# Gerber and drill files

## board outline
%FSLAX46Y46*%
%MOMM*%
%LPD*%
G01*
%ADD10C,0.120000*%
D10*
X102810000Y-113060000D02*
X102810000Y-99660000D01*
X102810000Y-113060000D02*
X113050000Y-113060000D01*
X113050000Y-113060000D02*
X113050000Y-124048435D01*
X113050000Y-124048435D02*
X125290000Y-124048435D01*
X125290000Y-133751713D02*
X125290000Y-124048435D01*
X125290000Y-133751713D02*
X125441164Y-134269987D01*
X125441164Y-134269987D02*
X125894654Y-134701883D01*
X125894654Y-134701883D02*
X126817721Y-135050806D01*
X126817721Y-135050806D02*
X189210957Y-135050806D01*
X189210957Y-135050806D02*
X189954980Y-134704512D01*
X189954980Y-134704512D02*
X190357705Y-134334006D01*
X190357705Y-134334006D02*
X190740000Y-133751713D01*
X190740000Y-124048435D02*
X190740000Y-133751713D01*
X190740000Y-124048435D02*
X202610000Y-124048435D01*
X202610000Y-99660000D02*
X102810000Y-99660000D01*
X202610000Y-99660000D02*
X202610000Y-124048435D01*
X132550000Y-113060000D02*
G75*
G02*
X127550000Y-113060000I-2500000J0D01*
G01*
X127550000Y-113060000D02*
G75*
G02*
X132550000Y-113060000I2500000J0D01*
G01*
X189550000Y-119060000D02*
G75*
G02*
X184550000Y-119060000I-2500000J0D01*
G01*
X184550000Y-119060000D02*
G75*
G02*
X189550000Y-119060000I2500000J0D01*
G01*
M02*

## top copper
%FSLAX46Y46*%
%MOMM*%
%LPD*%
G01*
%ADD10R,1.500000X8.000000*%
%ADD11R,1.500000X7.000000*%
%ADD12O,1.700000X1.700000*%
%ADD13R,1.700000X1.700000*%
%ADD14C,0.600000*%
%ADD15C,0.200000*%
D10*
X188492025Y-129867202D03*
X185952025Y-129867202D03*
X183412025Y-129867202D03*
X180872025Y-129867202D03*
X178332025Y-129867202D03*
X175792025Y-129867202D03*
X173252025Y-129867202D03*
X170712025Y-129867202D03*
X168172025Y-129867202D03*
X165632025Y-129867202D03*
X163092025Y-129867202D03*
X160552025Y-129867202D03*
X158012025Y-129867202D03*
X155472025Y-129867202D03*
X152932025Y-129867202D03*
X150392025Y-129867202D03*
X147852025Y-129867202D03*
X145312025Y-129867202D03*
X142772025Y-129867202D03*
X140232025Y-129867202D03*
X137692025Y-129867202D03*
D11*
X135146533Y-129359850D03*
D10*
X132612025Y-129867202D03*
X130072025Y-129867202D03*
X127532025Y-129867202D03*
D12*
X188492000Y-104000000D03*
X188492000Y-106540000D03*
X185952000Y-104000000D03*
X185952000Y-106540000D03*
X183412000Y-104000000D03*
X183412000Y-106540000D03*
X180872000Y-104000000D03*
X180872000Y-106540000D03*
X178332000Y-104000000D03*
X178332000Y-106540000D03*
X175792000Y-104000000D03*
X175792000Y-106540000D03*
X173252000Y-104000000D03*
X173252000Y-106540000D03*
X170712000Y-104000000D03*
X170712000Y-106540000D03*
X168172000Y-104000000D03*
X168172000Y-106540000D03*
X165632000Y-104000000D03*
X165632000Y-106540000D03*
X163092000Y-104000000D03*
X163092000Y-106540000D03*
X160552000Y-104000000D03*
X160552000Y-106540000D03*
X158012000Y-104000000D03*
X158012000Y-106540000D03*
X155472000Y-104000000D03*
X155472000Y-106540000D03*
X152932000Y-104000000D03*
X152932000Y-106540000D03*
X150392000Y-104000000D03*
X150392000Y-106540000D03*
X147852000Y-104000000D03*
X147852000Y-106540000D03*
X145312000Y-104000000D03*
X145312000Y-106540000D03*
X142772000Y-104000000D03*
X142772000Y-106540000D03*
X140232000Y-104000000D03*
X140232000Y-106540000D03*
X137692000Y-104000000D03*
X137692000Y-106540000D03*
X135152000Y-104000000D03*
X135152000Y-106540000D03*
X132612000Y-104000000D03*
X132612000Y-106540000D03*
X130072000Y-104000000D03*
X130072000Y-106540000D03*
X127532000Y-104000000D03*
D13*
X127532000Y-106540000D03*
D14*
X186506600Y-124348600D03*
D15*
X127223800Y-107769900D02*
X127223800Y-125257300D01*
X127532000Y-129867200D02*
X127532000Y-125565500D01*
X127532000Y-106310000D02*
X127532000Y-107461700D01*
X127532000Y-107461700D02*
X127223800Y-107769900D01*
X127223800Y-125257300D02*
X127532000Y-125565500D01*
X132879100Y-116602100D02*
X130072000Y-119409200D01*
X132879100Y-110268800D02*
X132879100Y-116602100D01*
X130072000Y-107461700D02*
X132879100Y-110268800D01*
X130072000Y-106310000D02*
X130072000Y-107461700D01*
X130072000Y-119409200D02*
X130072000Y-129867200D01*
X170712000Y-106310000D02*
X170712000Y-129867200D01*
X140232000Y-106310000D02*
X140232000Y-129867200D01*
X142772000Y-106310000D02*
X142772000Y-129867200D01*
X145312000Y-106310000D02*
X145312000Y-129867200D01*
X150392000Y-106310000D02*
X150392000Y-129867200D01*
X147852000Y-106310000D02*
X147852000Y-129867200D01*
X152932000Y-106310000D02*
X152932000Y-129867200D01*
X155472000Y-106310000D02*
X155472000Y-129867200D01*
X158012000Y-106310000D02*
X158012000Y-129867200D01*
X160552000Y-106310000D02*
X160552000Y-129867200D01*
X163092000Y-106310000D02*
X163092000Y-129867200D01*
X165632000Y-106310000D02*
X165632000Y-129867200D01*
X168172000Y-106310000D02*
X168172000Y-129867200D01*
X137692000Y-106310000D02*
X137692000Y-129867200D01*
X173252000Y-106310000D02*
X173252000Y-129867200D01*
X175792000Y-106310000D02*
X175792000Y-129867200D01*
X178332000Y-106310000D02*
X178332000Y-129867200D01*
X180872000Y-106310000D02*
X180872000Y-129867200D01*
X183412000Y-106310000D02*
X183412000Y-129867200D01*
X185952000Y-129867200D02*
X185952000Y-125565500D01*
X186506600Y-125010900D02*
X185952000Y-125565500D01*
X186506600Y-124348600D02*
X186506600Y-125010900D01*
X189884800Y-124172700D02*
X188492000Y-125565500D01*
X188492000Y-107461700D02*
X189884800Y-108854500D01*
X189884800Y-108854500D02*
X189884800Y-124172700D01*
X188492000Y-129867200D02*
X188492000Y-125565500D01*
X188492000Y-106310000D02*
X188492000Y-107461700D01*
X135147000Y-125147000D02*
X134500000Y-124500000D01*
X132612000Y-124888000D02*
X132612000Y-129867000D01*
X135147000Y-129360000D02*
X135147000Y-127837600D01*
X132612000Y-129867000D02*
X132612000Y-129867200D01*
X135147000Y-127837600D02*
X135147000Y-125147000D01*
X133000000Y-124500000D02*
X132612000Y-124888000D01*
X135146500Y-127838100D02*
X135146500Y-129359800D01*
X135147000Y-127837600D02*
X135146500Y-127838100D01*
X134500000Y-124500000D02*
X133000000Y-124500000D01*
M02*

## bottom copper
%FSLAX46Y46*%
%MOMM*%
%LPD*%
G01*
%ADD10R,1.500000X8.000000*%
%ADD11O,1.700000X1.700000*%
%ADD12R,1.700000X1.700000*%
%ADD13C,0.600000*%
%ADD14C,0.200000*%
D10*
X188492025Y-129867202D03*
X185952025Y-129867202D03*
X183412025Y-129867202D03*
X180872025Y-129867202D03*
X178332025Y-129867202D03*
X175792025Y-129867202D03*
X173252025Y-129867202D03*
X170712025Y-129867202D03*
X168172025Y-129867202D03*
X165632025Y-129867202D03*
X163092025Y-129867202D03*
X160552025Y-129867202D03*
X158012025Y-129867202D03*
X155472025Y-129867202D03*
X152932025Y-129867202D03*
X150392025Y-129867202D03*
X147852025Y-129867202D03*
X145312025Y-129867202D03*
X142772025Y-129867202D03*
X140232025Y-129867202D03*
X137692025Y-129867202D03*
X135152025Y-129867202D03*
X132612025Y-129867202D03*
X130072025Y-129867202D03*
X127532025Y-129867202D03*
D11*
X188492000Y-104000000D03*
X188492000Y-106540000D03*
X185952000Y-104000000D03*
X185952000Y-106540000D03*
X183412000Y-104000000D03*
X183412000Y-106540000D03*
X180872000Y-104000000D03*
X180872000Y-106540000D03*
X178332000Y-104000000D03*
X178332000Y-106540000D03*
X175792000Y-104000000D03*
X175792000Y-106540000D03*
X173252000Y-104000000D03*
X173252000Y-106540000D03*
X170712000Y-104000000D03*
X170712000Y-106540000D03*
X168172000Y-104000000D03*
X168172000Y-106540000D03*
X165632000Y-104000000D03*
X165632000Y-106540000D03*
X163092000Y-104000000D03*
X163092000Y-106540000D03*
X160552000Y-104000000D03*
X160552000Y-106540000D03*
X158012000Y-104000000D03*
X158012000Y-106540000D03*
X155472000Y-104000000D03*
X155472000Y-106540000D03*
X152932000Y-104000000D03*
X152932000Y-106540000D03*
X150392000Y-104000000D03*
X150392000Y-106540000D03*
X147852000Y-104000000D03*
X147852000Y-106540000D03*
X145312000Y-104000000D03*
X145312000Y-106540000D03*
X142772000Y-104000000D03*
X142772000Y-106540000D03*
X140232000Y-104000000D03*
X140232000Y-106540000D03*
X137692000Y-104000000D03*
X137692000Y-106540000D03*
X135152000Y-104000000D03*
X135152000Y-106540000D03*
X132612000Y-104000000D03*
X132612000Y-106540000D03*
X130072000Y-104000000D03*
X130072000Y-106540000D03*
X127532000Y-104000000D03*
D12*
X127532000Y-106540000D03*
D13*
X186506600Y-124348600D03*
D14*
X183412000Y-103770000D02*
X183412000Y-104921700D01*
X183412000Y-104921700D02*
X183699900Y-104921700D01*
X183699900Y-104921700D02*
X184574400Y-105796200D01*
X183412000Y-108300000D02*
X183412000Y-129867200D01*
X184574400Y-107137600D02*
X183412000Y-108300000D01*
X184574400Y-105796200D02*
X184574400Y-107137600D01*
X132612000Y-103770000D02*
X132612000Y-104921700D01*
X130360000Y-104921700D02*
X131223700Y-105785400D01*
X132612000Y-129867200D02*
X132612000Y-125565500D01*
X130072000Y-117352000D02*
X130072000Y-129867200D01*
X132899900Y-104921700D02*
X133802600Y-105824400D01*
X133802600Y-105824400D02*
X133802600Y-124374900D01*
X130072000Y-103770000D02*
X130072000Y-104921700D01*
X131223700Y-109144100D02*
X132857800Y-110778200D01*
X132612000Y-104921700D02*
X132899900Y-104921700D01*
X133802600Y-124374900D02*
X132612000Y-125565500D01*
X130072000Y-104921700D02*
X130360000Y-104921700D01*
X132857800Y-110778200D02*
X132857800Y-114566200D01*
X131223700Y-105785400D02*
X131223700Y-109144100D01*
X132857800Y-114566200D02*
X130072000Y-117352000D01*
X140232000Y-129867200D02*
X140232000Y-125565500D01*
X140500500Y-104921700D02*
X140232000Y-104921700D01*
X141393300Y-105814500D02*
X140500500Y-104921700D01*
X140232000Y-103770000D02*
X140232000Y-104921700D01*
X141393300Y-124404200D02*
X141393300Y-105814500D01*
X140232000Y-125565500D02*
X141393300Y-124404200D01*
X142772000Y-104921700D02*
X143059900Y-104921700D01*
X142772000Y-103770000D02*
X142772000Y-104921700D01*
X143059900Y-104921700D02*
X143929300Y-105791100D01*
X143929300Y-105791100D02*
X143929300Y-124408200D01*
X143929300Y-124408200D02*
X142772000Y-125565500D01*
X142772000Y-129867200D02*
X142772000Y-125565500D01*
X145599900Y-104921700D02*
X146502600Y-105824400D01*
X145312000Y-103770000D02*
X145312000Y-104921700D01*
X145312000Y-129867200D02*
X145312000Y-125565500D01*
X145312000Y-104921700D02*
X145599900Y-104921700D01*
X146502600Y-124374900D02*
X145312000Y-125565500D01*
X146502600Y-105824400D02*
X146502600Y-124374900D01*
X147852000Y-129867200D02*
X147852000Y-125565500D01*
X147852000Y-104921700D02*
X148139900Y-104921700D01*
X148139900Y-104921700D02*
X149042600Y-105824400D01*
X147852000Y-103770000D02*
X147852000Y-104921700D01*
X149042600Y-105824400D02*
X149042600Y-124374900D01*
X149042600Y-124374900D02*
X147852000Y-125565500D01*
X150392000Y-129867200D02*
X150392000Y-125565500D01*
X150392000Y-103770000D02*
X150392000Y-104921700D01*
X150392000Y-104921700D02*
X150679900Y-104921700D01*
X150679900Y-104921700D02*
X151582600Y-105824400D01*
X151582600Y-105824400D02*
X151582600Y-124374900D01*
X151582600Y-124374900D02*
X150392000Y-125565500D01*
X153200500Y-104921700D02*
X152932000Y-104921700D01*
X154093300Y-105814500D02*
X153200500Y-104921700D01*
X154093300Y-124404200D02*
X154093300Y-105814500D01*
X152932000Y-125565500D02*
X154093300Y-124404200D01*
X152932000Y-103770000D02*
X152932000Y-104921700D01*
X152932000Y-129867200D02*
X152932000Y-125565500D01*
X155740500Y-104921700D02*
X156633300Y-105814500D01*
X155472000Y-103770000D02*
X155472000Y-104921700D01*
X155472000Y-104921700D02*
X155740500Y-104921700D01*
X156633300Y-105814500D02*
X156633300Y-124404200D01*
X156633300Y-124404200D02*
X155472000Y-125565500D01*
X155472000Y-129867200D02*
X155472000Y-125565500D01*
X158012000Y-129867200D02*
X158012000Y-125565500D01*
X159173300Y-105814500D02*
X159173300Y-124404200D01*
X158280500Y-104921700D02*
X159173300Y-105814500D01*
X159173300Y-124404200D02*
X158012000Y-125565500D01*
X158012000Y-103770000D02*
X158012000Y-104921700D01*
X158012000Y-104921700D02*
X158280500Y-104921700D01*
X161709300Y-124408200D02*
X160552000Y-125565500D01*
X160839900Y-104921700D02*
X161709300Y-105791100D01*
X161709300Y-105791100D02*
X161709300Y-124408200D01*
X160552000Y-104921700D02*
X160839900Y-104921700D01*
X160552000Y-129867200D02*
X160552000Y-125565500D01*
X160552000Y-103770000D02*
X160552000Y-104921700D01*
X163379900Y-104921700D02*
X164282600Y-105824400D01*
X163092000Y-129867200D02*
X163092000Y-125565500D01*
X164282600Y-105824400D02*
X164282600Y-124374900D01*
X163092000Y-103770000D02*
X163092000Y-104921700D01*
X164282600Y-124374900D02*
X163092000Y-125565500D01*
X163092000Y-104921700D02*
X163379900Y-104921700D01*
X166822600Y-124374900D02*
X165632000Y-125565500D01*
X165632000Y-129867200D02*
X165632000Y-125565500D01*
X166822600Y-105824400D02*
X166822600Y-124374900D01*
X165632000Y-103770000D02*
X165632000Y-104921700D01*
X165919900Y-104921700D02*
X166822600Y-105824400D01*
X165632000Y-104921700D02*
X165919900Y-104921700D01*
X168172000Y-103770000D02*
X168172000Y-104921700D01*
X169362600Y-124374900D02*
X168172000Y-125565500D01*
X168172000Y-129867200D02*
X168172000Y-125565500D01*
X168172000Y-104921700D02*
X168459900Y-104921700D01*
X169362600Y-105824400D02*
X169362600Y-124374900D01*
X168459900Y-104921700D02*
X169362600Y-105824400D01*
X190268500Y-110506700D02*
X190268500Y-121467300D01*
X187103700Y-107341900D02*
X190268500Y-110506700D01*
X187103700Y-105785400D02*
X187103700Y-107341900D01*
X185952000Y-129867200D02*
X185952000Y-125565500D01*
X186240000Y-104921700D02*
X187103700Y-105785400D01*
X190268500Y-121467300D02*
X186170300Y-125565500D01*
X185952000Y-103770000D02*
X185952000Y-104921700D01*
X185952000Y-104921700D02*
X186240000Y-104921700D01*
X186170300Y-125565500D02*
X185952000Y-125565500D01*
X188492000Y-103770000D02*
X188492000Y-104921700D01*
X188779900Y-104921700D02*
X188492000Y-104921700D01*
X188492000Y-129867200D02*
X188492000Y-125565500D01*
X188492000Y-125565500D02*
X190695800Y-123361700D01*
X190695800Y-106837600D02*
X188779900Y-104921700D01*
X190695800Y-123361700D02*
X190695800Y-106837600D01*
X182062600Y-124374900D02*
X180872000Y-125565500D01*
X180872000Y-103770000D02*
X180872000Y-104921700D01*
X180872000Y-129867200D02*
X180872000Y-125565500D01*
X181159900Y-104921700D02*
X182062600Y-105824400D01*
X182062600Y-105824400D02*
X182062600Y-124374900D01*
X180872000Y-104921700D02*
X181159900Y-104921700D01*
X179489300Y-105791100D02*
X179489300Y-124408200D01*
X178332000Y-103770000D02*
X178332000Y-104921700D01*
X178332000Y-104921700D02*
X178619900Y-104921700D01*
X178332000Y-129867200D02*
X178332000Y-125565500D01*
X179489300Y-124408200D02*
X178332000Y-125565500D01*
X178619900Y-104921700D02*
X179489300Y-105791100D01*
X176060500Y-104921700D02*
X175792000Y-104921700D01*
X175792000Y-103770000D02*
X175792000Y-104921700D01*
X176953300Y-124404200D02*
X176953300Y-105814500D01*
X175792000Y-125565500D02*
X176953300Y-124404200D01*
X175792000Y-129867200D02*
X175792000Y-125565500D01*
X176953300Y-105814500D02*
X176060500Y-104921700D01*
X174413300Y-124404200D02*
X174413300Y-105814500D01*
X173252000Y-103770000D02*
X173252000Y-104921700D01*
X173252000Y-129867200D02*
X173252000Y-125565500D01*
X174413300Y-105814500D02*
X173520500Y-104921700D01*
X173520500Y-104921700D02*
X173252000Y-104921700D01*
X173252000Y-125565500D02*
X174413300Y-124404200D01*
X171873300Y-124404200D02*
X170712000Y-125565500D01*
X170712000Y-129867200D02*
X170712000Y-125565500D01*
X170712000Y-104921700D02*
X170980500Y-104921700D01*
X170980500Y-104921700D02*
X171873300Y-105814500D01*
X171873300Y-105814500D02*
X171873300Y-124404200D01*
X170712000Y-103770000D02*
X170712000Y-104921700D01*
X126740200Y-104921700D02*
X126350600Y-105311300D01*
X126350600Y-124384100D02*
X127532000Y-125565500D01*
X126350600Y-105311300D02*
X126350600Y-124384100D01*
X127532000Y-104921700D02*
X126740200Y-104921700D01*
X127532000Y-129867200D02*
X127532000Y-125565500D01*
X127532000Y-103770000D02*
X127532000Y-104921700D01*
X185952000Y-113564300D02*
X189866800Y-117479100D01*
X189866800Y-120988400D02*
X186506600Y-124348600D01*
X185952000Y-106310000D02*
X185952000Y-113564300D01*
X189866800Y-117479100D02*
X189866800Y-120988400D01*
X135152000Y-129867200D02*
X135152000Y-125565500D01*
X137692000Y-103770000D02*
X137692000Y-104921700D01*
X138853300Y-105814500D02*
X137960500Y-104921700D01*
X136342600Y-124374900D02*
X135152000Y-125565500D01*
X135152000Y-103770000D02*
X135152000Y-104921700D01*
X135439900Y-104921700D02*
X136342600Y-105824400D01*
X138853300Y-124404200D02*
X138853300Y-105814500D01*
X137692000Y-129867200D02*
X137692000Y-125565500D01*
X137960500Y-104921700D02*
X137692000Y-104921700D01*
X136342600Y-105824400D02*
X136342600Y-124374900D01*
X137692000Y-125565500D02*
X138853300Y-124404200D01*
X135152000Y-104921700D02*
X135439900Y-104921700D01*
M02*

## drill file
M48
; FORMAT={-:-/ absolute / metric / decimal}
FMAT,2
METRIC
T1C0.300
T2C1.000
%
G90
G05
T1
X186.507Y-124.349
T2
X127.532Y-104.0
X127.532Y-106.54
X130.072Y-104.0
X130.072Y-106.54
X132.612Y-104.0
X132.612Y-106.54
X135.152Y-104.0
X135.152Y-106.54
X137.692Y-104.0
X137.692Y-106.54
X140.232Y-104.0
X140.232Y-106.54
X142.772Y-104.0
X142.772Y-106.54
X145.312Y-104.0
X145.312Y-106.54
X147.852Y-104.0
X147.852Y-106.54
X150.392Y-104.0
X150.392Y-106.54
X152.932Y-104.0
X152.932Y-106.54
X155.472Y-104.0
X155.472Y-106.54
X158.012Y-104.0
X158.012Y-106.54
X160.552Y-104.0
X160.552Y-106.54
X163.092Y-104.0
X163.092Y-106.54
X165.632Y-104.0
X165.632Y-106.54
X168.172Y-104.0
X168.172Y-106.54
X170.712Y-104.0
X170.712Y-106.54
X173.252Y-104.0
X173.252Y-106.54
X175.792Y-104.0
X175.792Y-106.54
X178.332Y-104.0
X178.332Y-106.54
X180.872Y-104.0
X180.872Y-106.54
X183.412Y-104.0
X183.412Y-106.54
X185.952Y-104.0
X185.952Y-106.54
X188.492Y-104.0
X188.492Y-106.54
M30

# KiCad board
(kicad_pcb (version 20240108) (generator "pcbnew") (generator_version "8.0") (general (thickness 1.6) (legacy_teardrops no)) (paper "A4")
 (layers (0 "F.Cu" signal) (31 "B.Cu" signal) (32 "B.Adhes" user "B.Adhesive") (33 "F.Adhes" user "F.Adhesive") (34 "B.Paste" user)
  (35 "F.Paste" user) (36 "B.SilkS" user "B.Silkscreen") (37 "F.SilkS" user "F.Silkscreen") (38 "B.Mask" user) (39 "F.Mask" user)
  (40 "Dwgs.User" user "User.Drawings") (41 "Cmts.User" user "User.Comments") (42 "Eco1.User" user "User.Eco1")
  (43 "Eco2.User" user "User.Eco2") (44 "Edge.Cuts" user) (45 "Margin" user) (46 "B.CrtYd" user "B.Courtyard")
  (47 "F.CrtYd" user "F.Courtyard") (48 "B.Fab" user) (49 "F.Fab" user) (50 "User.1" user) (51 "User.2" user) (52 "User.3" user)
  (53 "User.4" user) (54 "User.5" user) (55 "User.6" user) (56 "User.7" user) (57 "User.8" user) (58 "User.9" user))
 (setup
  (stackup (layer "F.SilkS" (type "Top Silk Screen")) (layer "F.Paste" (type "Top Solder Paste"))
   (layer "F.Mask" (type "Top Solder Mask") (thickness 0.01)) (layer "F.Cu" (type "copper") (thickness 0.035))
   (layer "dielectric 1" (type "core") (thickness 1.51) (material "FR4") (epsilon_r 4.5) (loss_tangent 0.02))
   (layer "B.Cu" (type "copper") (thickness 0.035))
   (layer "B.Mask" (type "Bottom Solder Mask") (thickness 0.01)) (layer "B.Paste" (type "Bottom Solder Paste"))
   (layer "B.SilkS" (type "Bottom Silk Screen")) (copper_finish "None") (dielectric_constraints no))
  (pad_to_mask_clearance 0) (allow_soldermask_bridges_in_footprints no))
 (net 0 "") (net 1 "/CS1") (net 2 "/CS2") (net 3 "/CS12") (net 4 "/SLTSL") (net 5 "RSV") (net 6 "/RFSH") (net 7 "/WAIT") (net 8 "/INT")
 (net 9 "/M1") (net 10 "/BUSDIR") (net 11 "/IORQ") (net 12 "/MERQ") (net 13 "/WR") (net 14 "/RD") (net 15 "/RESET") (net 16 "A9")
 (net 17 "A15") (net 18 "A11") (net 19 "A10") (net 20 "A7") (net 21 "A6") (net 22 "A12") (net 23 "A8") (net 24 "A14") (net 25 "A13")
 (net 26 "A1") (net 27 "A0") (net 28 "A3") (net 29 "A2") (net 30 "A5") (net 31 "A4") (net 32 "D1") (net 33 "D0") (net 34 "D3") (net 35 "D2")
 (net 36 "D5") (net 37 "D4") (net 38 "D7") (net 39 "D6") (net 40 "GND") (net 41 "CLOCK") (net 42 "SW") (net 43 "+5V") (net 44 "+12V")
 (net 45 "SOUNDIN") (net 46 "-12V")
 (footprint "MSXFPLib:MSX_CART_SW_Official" (layer "F.Cu") (at 151.71 99.66)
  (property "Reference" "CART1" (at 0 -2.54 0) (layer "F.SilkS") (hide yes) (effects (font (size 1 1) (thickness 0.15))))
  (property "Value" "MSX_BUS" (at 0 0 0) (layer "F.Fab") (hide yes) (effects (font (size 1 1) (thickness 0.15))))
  (fp_line (start -48.9 13.4) (end -48.9 0) (stroke (width 0.12) (type solid)) (layer "Edge.Cuts"))
  (fp_line (start -48.9 13.4) (end -38.66 13.4) (stroke (width 0.12) (type solid)) (layer "Edge.Cuts"))
  (fp_line (start -38.66 13.4) (end -38.66 24.388435) (stroke (width 0.12) (type solid)) (layer "Edge.Cuts"))
  (fp_line (start -38.66 24.388435) (end -26.42 24.388435) (stroke (width 0.12) (type solid)) (layer "Edge.Cuts"))
  (fp_line (start -26.42 34.091713) (end -26.42 24.388435) (stroke (width 0.12) (type solid)) (layer "Edge.Cuts"))
  (fp_line (start -26.42 34.091713) (end -26.268836 34.609987) (stroke (width 0.12) (type solid)) (layer "Edge.Cuts"))
  (fp_line (start -26.268836 34.609987) (end -25.815346 35.041883) (stroke (width 0.12) (type solid)) (layer "Edge.Cuts"))
  (fp_line (start -25.815346 35.041883) (end -24.892279 35.390806) (stroke (width 0.12) (type solid)) (layer "Edge.Cuts"))
  (fp_line (start -24.892279 35.390806) (end 37.500957 35.390806) (stroke (width 0.12) (type solid)) (layer "Edge.Cuts"))
  (fp_line (start 37.500957 35.390806) (end 38.24498 35.044512) (stroke (width 0.12) (type solid)) (layer "Edge.Cuts"))
  (fp_line (start 38.24498 35.044512) (end 38.647705 34.674006) (stroke (width 0.12) (type solid)) (layer "Edge.Cuts"))
  (fp_line (start 38.647705 34.674006) (end 39.03 34.091713) (stroke (width 0.12) (type solid)) (layer "Edge.Cuts"))
  (fp_line (start 39.03 24.388435) (end 39.03 34.091713) (stroke (width 0.12) (type solid)) (layer "Edge.Cuts"))
  (fp_line (start 39.03 24.388435) (end 50.9 24.388435) (stroke (width 0.12) (type solid)) (layer "Edge.Cuts"))
  (fp_line (start 50.9 0) (end -48.9 0) (stroke (width 0.12) (type solid)) (layer "Edge.Cuts"))
  (fp_line (start 50.9 0) (end 50.9 24.388435) (stroke (width 0.12) (type solid)) (layer "Edge.Cuts"))
  (fp_circle (center -21.66 13.4) (end -19.16 13.4) (stroke (width 0.12) (type solid)) (fill none) (layer "Edge.Cuts"))
  (fp_circle (center 35.34 19.4) (end 37.84 19.4) (stroke (width 0.12) (type solid)) (fill none) (layer "Edge.Cuts"))
  (pad "1" connect rect (at 36.782025 30.207202) (size 1.5 8) (layers "B.Cu" "B.Mask") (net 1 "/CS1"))
  (pad "2" connect rect (at 36.782025 30.207202) (size 1.5 8) (layers "F.Cu" "F.Mask") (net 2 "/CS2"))
  (pad "3" connect rect (at 34.242025 30.207202) (size 1.5 8) (layers "B.Cu" "B.Mask") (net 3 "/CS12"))
  (pad "4" connect rect (at 34.242025 30.207202) (size 1.5 8) (layers "F.Cu" "F.Mask") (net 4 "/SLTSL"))
  (pad "5" connect rect (at 31.702025 30.207202) (size 1.5 8) (layers "B.Cu" "B.Mask") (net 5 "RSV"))
  (pad "6" connect rect (at 31.702025 30.207202) (size 1.5 8) (layers "F.Cu" "F.Mask") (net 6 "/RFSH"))
  (pad "7" connect rect (at 29.162025 30.207202) (size 1.5 8) (layers "B.Cu" "B.Mask") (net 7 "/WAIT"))
  (pad "8" connect rect (at 29.162025 30.207202) (size 1.5 8) (layers "F.Cu" "F.Mask") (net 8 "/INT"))
  (pad "9" connect rect (at 26.622025 30.207202) (size 1.5 8) (layers "B.Cu" "B.Mask") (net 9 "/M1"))
  (pad "10" connect rect (at 26.622025 30.207202) (size 1.5 8) (layers "F.Cu" "F.Mask") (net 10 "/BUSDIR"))
  (pad "11" connect rect (at 24.082025 30.207202) (size 1.5 8) (layers "B.Cu" "B.Mask") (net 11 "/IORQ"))
  (pad "12" connect rect (at 24.082025 30.207202) (size 1.5 8) (layers "F.Cu" "F.Mask") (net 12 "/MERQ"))
  (pad "13" connect rect (at 21.542025 30.207202) (size 1.5 8) (layers "B.Cu" "B.Mask") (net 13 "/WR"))
  (pad "14" connect rect (at 21.542025 30.207202) (size 1.5 8) (layers "F.Cu" "F.Mask") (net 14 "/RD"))
  (pad "15" connect rect (at 19.002025 30.207202) (size 1.5 8) (layers "B.Cu" "B.Mask") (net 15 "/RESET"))
  (pad "16" connect rect (at 19.002025 30.207202) (size 1.5 8) (layers "F.Cu" "F.Mask") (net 5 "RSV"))
  (pad "17" connect rect (at 16.462025 30.207202) (size 1.5 8) (layers "B.Cu" "B.Mask") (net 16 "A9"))
  (pad "18" connect rect (at 16.462025 30.207202) (size 1.5 8) (layers "F.Cu" "F.Mask") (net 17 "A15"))
  (pad "19" connect rect (at 13.922025 30.207202) (size 1.5 8) (layers "B.Cu" "B.Mask") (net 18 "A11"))
  (pad "20" connect rect (at 13.922025 30.207202) (size 1.5 8) (layers "F.Cu" "F.Mask") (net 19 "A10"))
  (pad "21" connect rect (at 11.382025 30.207202) (size 1.5 8) (layers "B.Cu" "B.Mask") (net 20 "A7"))
  (pad "22" connect rect (at 11.382025 30.207202) (size 1.5 8) (layers "F.Cu" "F.Mask") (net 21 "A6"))
  (pad "23" connect rect (at 8.842025 30.207202) (size 1.5 8) (layers "B.Cu" "B.Mask") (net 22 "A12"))
  (pad "24" connect rect (at 8.842025 30.207202) (size 1.5 8) (layers "F.Cu" "F.Mask") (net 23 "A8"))
  (pad "25" connect rect (at 6.302025 30.207202) (size 1.5 8) (layers "B.Cu" "B.Mask") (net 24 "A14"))
  (pad "26" connect rect (at 6.302025 30.207202) (size 1.5 8) (layers "F.Cu" "F.Mask") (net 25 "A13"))
  (pad "27" connect rect (at 3.762025 30.207202) (size 1.5 8) (layers "B.Cu" "B.Mask") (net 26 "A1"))
  (pad "28" connect rect (at 3.762025 30.207202) (size 1.5 8) (layers "F.Cu" "F.Mask") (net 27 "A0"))
  (pad "29" connect rect (at 1.222025 30.207202) (size 1.5 8) (layers "B.Cu" "B.Mask") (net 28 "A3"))
  (pad "30" connect rect (at 1.222025 30.207202) (size 1.5 8) (layers "F.Cu" "F.Mask") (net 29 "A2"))
  (pad "31" connect rect (at -1.317975 30.207202) (size 1.5 8) (layers "B.Cu" "B.Mask") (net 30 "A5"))
  (pad "32" connect rect (at -1.317975 30.207202) (size 1.5 8) (layers "F.Cu" "F.Mask") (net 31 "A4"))
  (pad "33" connect rect (at -3.857975 30.207202) (size 1.5 8) (layers "B.Cu" "B.Mask") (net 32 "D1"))
  (pad "34" connect rect (at -3.857975 30.207202) (size 1.5 8) (layers "F.Cu" "F.Mask") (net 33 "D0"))
  (pad "35" connect rect (at -6.397975 30.207202) (size 1.5 8) (layers "B.Cu" "B.Mask") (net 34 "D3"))
  (pad "36" connect rect (at -6.397975 30.207202) (size 1.5 8) (layers "F.Cu" "F.Mask") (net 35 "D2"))
  (pad "37" connect rect (at -8.937975 30.207202) (size 1.5 8) (layers "B.Cu" "B.Mask") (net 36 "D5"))
  (pad "38" connect rect (at -8.937975 30.207202) (size 1.5 8) (layers "F.Cu" "F.Mask") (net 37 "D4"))
  (pad "39" connect rect (at -11.477975 30.207202) (size 1.5 8) (layers "B.Cu" "B.Mask") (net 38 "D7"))
  (pad "40" connect rect (at -11.477975 30.207202) (size 1.5 8) (layers "F.Cu" "F.Mask") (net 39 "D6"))
  (pad "41" connect rect (at -14.017975 30.207202) (size 1.5 8) (layers "B.Cu" "B.Mask") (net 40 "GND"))
  (pad "42" connect rect (at -14.017975 30.207202) (size 1.5 8) (layers "F.Cu" "F.Mask") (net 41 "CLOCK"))
  (pad "43" connect rect (at -16.557975 30.207202) (size 1.5 8) (layers "B.Cu" "B.Mask") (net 40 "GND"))
  (pad "44" connect rect (at -16.563467 29.69985) (size 1.5 7) (layers "F.Cu" "F.Mask") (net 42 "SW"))
  (pad "45" connect rect (at -19.097975 30.207202) (size 1.5 8) (layers "B.Cu" "B.Mask") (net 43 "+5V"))
  (pad "46" connect rect (at -19.097975 30.207202) (size 1.5 8) (layers "F.Cu" "F.Mask") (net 42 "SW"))
  (pad "47" connect rect (at -21.637975 30.207202) (size 1.5 8) (layers "B.Cu" "B.Mask") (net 43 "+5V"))
  (pad "48" connect rect (at -21.637975 30.207202) (size 1.5 8) (layers "F.Cu" "F.Mask") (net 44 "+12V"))
  (pad "49" connect rect (at -24.177975 30.207202) (size 1.5 8) (layers "B.Cu" "B.Mask") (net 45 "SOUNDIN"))
  (pad "50" connect rect (at -24.177975 30.207202) (size 1.5 8) (layers "F.Cu" "F.Mask") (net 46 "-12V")))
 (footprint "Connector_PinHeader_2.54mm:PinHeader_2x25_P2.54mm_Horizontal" (layer "F.Cu") (at 127.532 106.54 90)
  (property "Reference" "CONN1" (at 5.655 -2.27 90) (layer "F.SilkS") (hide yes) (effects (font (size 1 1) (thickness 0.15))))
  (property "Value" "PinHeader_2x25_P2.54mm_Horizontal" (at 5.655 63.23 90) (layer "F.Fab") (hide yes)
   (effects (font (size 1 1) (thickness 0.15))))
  (pad "1" thru_hole oval (at 2.54 60.96 90) (size 1.7 1.7) (drill 1) (layers "*.Cu" "*.Mask") (remove_unused_layers no) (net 1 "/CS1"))
  (pad "2" thru_hole oval (at 0 60.96 90) (size 1.7 1.7) (drill 1) (layers "*.Cu" "*.Mask") (remove_unused_layers no) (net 2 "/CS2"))
  (pad "3" thru_hole oval (at 2.54 58.42 90) (size 1.7 1.7) (drill 1) (layers "*.Cu" "*.Mask") (remove_unused_layers no) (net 3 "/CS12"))
  (pad "4" thru_hole oval (at 0 58.42 90) (size 1.7 1.7) (drill 1) (layers "*.Cu" "*.Mask") (remove_unused_layers no) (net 4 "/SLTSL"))
  (pad "5" thru_hole oval (at 2.54 55.88 90) (size 1.7 1.7) (drill 1) (layers "*.Cu" "*.Mask") (remove_unused_layers no) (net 5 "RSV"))
  (pad "6" thru_hole oval (at 0 55.88 90) (size 1.7 1.7) (drill 1) (layers "*.Cu" "*.Mask") (remove_unused_layers no) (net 6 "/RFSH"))
  (pad "7" thru_hole oval (at 2.54 53.34 90) (size 1.7 1.7) (drill 1) (layers "*.Cu" "*.Mask") (remove_unused_layers no) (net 7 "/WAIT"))
  (pad "8" thru_hole oval (at 0 53.34 90) (size 1.7 1.7) (drill 1) (layers "*.Cu" "*.Mask") (remove_unused_layers no) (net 8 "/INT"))
  (pad "9" thru_hole oval (at 2.54 50.8 90) (size 1.7 1.7) (drill 1) (layers "*.Cu" "*.Mask") (remove_unused_layers no) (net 9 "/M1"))
  (pad "10" thru_hole oval (at 0 50.8 90) (size 1.7 1.7) (drill 1) (layers "*.Cu" "*.Mask") (remove_unused_layers no) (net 10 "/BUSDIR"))
  (pad "11" thru_hole oval (at 2.54 48.26 90) (size 1.7 1.7) (drill 1) (layers "*.Cu" "*.Mask") (remove_unused_layers no) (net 11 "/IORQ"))
  (pad "12" thru_hole oval (at 0 48.26 90) (size 1.7 1.7) (drill 1) (layers "*.Cu" "*.Mask") (remove_unused_layers no) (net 12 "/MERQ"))
  (pad "13" thru_hole oval (at 2.54 45.72 90) (size 1.7 1.7) (drill 1) (layers "*.Cu" "*.Mask") (remove_unused_layers no) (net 13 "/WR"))
  (pad "14" thru_hole oval (at 0 45.72 90) (size 1.7 1.7) (drill 1) (layers "*.Cu" "*.Mask") (remove_unused_layers no) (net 14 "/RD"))
  (pad "15" thru_hole oval (at 2.54 43.18 90) (size 1.7 1.7) (drill 1) (layers "*.Cu" "*.Mask") (remove_unused_layers no) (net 15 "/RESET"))
  (pad "16" thru_hole oval (at 0 43.18 90) (size 1.7 1.7) (drill 1) (layers "*.Cu" "*.Mask") (remove_unused_layers no) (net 5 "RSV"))
  (pad "17" thru_hole oval (at 2.54 40.64 90) (size 1.7 1.7) (drill 1) (layers "*.Cu" "*.Mask") (remove_unused_layers no) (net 16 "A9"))
  (pad "18" thru_hole oval (at 0 40.64 90) (size 1.7 1.7) (drill 1) (layers "*.Cu" "*.Mask") (remove_unused_layers no) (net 17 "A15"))
  (pad "19" thru_hole oval (at 2.54 38.1 90) (size 1.7 1.7) (drill 1) (layers "*.Cu" "*.Mask") (remove_unused_layers no) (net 18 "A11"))
  (pad "20" thru_hole oval (at 0 38.1 90) (size 1.7 1.7) (drill 1) (layers "*.Cu" "*.Mask") (remove_unused_layers no) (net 19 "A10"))
  (pad "21" thru_hole oval (at 2.54 35.56 90) (size 1.7 1.7) (drill 1) (layers "*.Cu" "*.Mask") (remove_unused_layers no) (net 20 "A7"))
  (pad "22" thru_hole oval (at 0 35.56 90) (size 1.7 1.7) (drill 1) (layers "*.Cu" "*.Mask") (remove_unused_layers no) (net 21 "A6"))
  (pad "23" thru_hole oval (at 2.54 33.02 90) (size 1.7 1.7) (drill 1) (layers "*.Cu" "*.Mask") (remove_unused_layers no) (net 22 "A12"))
  (pad "24" thru_hole oval (at 0 33.02 90) (size 1.7 1.7) (drill 1) (layers "*.Cu" "*.Mask") (remove_unused_layers no) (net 23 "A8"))
  (pad "25" thru_hole oval (at 2.54 30.48 90) (size 1.7 1.7) (drill 1) (layers "*.Cu" "*.Mask") (remove_unused_layers no) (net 24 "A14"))
  (pad "26" thru_hole oval (at 0 30.48 90) (size 1.7 1.7) (drill 1) (layers "*.Cu" "*.Mask") (remove_unused_layers no) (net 25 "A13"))
  (pad "27" thru_hole oval (at 2.54 27.94 90) (size 1.7 1.7) (drill 1) (layers "*.Cu" "*.Mask") (remove_unused_layers no) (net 26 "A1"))
  (pad "28" thru_hole oval (at 0 27.94 90) (size 1.7 1.7) (drill 1) (layers "*.Cu" "*.Mask") (remove_unused_layers no) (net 27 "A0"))
  (pad "29" thru_hole oval (at 2.54 25.4 90) (size 1.7 1.7) (drill 1) (layers "*.Cu" "*.Mask") (remove_unused_layers no) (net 28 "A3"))
  (pad "30" thru_hole oval (at 0 25.4 90) (size 1.7 1.7) (drill 1) (layers "*.Cu" "*.Mask") (remove_unused_layers no) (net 29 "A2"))
  (pad "31" thru_hole oval (at 2.54 22.86 90) (size 1.7 1.7) (drill 1) (layers "*.Cu" "*.Mask") (remove_unused_layers no) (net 30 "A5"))
  (pad "32" thru_hole oval (at 0 22.86 90) (size 1.7 1.7) (drill 1) (layers "*.Cu" "*.Mask") (remove_unused_layers no) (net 31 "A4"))
  (pad "33" thru_hole oval (at 2.54 20.32 90) (size 1.7 1.7) (drill 1) (layers "*.Cu" "*.Mask") (remove_unused_layers no) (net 32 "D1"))
  (pad "34" thru_hole oval (at 0 20.32 90) (size 1.7 1.7) (drill 1) (layers "*.Cu" "*.Mask") (remove_unused_layers no) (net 33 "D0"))
  (pad "35" thru_hole oval (at 2.54 17.78 90) (size 1.7 1.7) (drill 1) (layers "*.Cu" "*.Mask") (remove_unused_layers no) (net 34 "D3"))
  (pad "36" thru_hole oval (at 0 17.78 90) (size 1.7 1.7) (drill 1) (layers "*.Cu" "*.Mask") (remove_unused_layers no) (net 35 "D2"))
  (pad "37" thru_hole oval (at 2.54 15.24 90) (size 1.7 1.7) (drill 1) (layers "*.Cu" "*.Mask") (remove_unused_layers no) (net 36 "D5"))
  (pad "38" thru_hole oval (at 0 15.24 90) (size 1.7 1.7) (drill 1) (layers "*.Cu" "*.Mask") (remove_unused_layers no) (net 37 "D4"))
  (pad "39" thru_hole oval (at 2.54 12.7 90) (size 1.7 1.7) (drill 1) (layers "*.Cu" "*.Mask") (remove_unused_layers no) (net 38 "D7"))
  (pad "40" thru_hole oval (at 0 12.7 90) (size 1.7 1.7) (drill 1) (layers "*.Cu" "*.Mask") (remove_unused_layers no) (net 39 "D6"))
  (pad "41" thru_hole oval (at 2.54 10.16 90) (size 1.7 1.7) (drill 1) (layers "*.Cu" "*.Mask") (remove_unused_layers no) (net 40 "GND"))
  (pad "42" thru_hole oval (at 0 10.16 90) (size 1.7 1.7) (drill 1) (layers "*.Cu" "*.Mask") (remove_unused_layers no) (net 41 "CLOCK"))
  (pad "43" thru_hole oval (at 2.54 7.62 90) (size 1.7 1.7) (drill 1) (layers "*.Cu" "*.Mask") (remove_unused_layers no) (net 40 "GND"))
  (pad "44" thru_hole oval (at 0 7.62 90) (size 1.7 1.7) (drill 1) (layers "*.Cu" "*.Mask") (remove_unused_layers no) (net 42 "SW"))
  (pad "45" thru_hole oval (at 2.54 5.08 90) (size 1.7 1.7) (drill 1) (layers "*.Cu" "*.Mask") (remove_unused_layers no) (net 43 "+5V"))
  (pad "46" thru_hole oval (at 0 5.08 90) (size 1.7 1.7) (drill 1) (layers "*.Cu" "*.Mask") (remove_unused_layers no) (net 42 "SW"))
  (pad "47" thru_hole oval (at 2.54 2.54 90) (size 1.7 1.7) (drill 1) (layers "*.Cu" "*.Mask") (remove_unused_layers no) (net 43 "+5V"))
  (pad "48" thru_hole oval (at 0 2.54 90) (size 1.7 1.7) (drill 1) (layers "*.Cu" "*.Mask") (remove_unused_layers no) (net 44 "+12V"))
  (pad "49" thru_hole oval (at 2.54 0 90) (size 1.7 1.7) (drill 1) (layers "*.Cu" "*.Mask") (remove_unused_layers no) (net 45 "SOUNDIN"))
  (pad "50" thru_hole rect (at 0 0 90) (size 1.7 1.7) (drill 1) (layers "*.Cu" "*.Mask") (remove_unused_layers no) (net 46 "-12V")))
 (segment (start 127.2238 107.7699) (end 127.2238 125.2573) (width 0.2) (layer "F.Cu") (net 46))
 (segment (start 127.532 129.8672) (end 127.532 125.5655) (width 0.2) (layer "F.Cu") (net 46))
 (segment (start 127.532 106.31) (end 127.532 107.4617) (width 0.2) (layer "F.Cu") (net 46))
 (segment (start 127.532 107.4617) (end 127.2238 107.7699) (width 0.2) (layer "F.Cu") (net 46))
 (segment (start 127.2238 125.2573) (end 127.532 125.5655) (width 0.2) (layer "F.Cu") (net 46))
 (segment (start 132.8791 116.6021) (end 130.072 119.4092) (width 0.2) (layer "F.Cu") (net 44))
 (segment (start 132.8791 110.2688) (end 132.8791 116.6021) (width 0.2) (layer "F.Cu") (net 44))
 (segment (start 130.072 107.4617) (end 132.8791 110.2688) (width 0.2) (layer "F.Cu") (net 44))
 (segment (start 130.072 106.31) (end 130.072 107.4617) (width 0.2) (layer "F.Cu") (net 44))
 (segment (start 130.072 119.4092) (end 130.072 129.8672) (width 0.2) (layer "F.Cu") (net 44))
 (segment (start 170.712 106.31) (end 170.712 129.8672) (width 0.2) (layer "F.Cu") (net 5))
 (segment (start 183.412 103.77) (end 183.412 104.9217) (width 0.2) (layer "B.Cu") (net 5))
 (segment (start 183.412 104.9217) (end 183.6999 104.9217) (width 0.2) (layer "B.Cu") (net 5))
 (segment (start 183.6999 104.9217) (end 184.5744 105.7962) (width 0.2) (layer "B.Cu") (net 5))
 (segment (start 183.412 108.3) (end 183.412 129.8672) (width 0.2) (layer "B.Cu") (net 5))
 (segment (start 184.5744 107.1376) (end 183.412 108.3) (width 0.2) (layer "B.Cu") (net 5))
 (segment (start 184.5744 105.7962) (end 184.5744 107.1376) (width 0.2) (layer "B.Cu") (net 5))
 (segment (start 140.232 106.31) (end 140.232 129.8672) (width 0.2) (layer "F.Cu") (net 39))
 (segment (start 142.772 106.31) (end 142.772 129.8672) (width 0.2) (layer "F.Cu") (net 37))
 (segment (start 145.312 106.31) (end 145.312 129.8672) (width 0.2) (layer "F.Cu") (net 35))
 (segment (start 150.392 106.31) (end 150.392 129.8672) (width 0.2) (layer "F.Cu") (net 31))
 (segment (start 147.852 106.31) (end 147.852 129.8672) (width 0.2) (layer "F.Cu") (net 33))
 (segment (start 152.932 106.31) (end 152.932 129.8672) (width 0.2) (layer "F.Cu") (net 29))
 (segment (start 155.472 106.31) (end 155.472 129.8672) (width 0.2) (layer "F.Cu") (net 27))
 (segment (start 158.012 106.31) (end 158.012 129.8672) (width 0.2) (layer "F.Cu") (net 25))
 (segment (start 160.552 106.31) (end 160.552 129.8672) (width 0.2) (layer "F.Cu") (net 23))
 (segment (start 163.092 106.31) (end 163.092 129.8672) (width 0.2) (layer "F.Cu") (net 21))
 (segment (start 165.632 106.31) (end 165.632 129.8672) (width 0.2) (layer "F.Cu") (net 19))
 (segment (start 168.172 106.31) (end 168.172 129.8672) (width 0.2) (layer "F.Cu") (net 17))
 (segment (start 132.612 103.77) (end 132.612 104.9217) (width 0.2) (layer "B.Cu") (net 43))
 (segment (start 130.36 104.9217) (end 131.2237 105.7854) (width 0.2) (layer "B.Cu") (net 43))
 (segment (start 132.612 129.8672) (end 132.612 125.5655) (width 0.2) (layer "B.Cu") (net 43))
 (segment (start 130.072 117.352) (end 130.072 129.8672) (width 0.2) (layer "B.Cu") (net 43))
 (segment (start 132.8999 104.9217) (end 133.8026 105.8244) (width 0.2) (layer "B.Cu") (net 43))
 (segment (start 133.8026 105.8244) (end 133.8026 124.3749) (width 0.2) (layer "B.Cu") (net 43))
 (segment (start 130.072 103.77) (end 130.072 104.9217) (width 0.2) (layer "B.Cu") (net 43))
 (segment (start 131.2237 109.1441) (end 132.8578 110.7782) (width 0.2) (layer "B.Cu") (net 43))
 (segment (start 132.612 104.9217) (end 132.8999 104.9217) (width 0.2) (layer "B.Cu") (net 43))
 (segment (start 133.8026 124.3749) (end 132.612 125.5655) (width 0.2) (layer "B.Cu") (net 43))
 (segment (start 130.072 104.9217) (end 130.36 104.9217) (width 0.2) (layer "B.Cu") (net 43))
 (segment (start 132.8578 110.7782) (end 132.8578 114.5662) (width 0.2) (layer "B.Cu") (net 43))
 (segment (start 131.2237 105.7854) (end 131.2237 109.1441) (width 0.2) (layer "B.Cu") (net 43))
 (segment (start 132.8578 114.5662) (end 130.072 117.352) (width 0.2) (layer "B.Cu") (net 43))
 (segment (start 140.232 129.8672) (end 140.232 125.5655) (width 0.2) (layer "B.Cu") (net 38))
 (segment (start 140.5005 104.9217) (end 140.232 104.9217) (width 0.2) (layer "B.Cu") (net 38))
 (segment (start 141.3933 105.8145) (end 140.5005 104.9217) (width 0.2) (layer "B.Cu") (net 38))
 (segment (start 140.232 103.77) (end 140.232 104.9217) (width 0.2) (layer "B.Cu") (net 38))
 (segment (start 141.3933 124.4042) (end 141.3933 105.8145) (width 0.2) (layer "B.Cu") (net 38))
 (segment (start 140.232 125.5655) (end 141.3933 124.4042) (width 0.2) (layer "B.Cu") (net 38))
 (segment (start 142.772 104.9217) (end 143.0599 104.9217) (width 0.2) (layer "B.Cu") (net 36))
 (segment (start 142.772 103.77) (end 142.772 104.9217) (width 0.2) (layer "B.Cu") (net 36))
 (segment (start 143.0599 104.9217) (end 143.9293 105.7911) (width 0.2) (layer "B.Cu") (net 36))
 (segment (start 143.9293 105.7911) (end 143.9293 124.4082) (width 0.2) (layer "B.Cu") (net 36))
 (segment (start 143.9293 124.4082) (end 142.772 125.5655) (width 0.2) (layer "B.Cu") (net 36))
 (segment (start 142.772 129.8672) (end 142.772 125.5655) (width 0.2) (layer "B.Cu") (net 36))
 (segment (start 145.5999 104.9217) (end 146.5026 105.8244) (width 0.2) (layer "B.Cu") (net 34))
 (segment (start 145.312 103.77) (end 145.312 104.9217) (width 0.2) (layer "B.Cu") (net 34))
 (segment (start 145.312 129.8672) (end 145.312 125.5655) (width 0.2) (layer "B.Cu") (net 34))
 (segment (start 145.312 104.9217) (end 145.5999 104.9217) (width 0.2) (layer "B.Cu") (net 34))
 (segment (start 146.5026 124.3749) (end 145.312 125.5655) (width 0.2) (layer "B.Cu") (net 34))
 (segment (start 146.5026 105.8244) (end 146.5026 124.3749) (width 0.2) (layer "B.Cu") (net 34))
 (segment (start 147.852 129.8672) (end 147.852 125.5655) (width 0.2) (layer "B.Cu") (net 32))
 (segment (start 147.852 104.9217) (end 148.1399 104.9217) (width 0.2) (layer "B.Cu") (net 32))
 (segment (start 148.1399 104.9217) (end 149.0426 105.8244) (width 0.2) (layer "B.Cu") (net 32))
 (segment (start 147.852 103.77) (end 147.852 104.9217) (width 0.2) (layer "B.Cu") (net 32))
 (segment (start 149.0426 105.8244) (end 149.0426 124.3749) (width 0.2) (layer "B.Cu") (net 32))
 (segment (start 149.0426 124.3749) (end 147.852 125.5655) (width 0.2) (layer "B.Cu") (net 32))
 (segment (start 150.392 129.8672) (end 150.392 125.5655) (width 0.2) (layer "B.Cu") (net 30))
 (segment (start 150.392 103.77) (end 150.392 104.9217) (width 0.2) (layer "B.Cu") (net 30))
 (segment (start 150.392 104.9217) (end 150.6799 104.9217) (width 0.2) (layer "B.Cu") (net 30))
 (segment (start 150.6799 104.9217) (end 151.5826 105.8244) (width 0.2) (layer "B.Cu") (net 30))
 (segment (start 151.5826 105.8244) (end 151.5826 124.3749) (width 0.2) (layer "B.Cu") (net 30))
 (segment (start 151.5826 124.3749) (end 150.392 125.5655) (width 0.2) (layer "B.Cu") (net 30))
 (segment (start 153.2005 104.9217) (end 152.932 104.9217) (width 0.2) (layer "B.Cu") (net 28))
 (segment (start 154.0933 105.8145) (end 153.2005 104.9217) (width 0.2) (layer "B.Cu") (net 28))
 (segment (start 154.0933 124.4042) (end 154.0933 105.8145) (width 0.2) (layer "B.Cu") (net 28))
 (segment (start 152.932 125.5655) (end 154.0933 124.4042) (width 0.2) (layer "B.Cu") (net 28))
 (segment (start 152.932 103.77) (end 152.932 104.9217) (width 0.2) (layer "B.Cu") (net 28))
 (segment (start 152.932 129.8672) (end 152.932 125.5655) (width 0.2) (layer "B.Cu") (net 28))
 (segment (start 155.7405 104.9217) (end 156.6333 105.8145) (width 0.2) (layer "B.Cu") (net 26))
 (segment (start 155.472 103.77) (end 155.472 104.9217) (width 0.2) (layer "B.Cu") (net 26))
 (segment (start 155.472 104.9217) (end 155.7405 104.9217) (width 0.2) (layer "B.Cu") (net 26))
 (segment (start 156.6333 105.8145) (end 156.6333 124.4042) (width 0.2) (layer "B.Cu") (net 26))
 (segment (start 156.6333 124.4042) (end 155.472 125.5655) (width 0.2) (layer "B.Cu") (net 26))
 (segment (start 155.472 129.8672) (end 155.472 125.5655) (width 0.2) (layer "B.Cu") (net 26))
 (segment (start 158.012 129.8672) (end 158.012 125.5655) (width 0.2) (layer "B.Cu") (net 24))
 (segment (start 159.1733 105.8145) (end 159.1733 124.4042) (width 0.2) (layer "B.Cu") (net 24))
 (segment (start 158.2805 104.9217) (end 159.1733 105.8145) (width 0.2) (layer "B.Cu") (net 24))
 (segment (start 159.1733 124.4042) (end 158.012 125.5655) (width 0.2) (layer "B.Cu") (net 24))
 (segment (start 158.012 103.77) (end 158.012 104.9217) (width 0.2) (layer "B.Cu") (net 24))
 (segment (start 158.012 104.9217) (end 158.2805 104.9217) (width 0.2) (layer "B.Cu") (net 24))
 (segment (start 161.7093 124.4082) (end 160.552 125.5655) (width 0.2) (layer "B.Cu") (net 22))
 (segment (start 160.8399 104.9217) (end 161.7093 105.7911) (width 0.2) (layer "B.Cu") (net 22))
 (segment (start 161.7093 105.7911) (end 161.7093 124.4082) (width 0.2) (layer "B.Cu") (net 22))
 (segment (start 160.552 104.9217) (end 160.8399 104.9217) (width 0.2) (layer "B.Cu") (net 22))
 (segment (start 160.552 129.8672) (end 160.552 125.5655) (width 0.2) (layer "B.Cu") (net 22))
 (segment (start 160.552 103.77) (end 160.552 104.9217) (width 0.2) (layer "B.Cu") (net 22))
 (segment (start 163.3799 104.9217) (end 164.2826 105.8244) (width 0.2) (layer "B.Cu") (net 20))
 (segment (start 163.092 129.8672) (end 163.092 125.5655) (width 0.2) (layer "B.Cu") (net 20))
 (segment (start 164.2826 105.8244) (end 164.2826 124.3749) (width 0.2) (layer "B.Cu") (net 20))
 (segment (start 163.092 103.77) (end 163.092 104.9217) (width 0.2) (layer "B.Cu") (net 20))
 (segment (start 164.2826 124.3749) (end 163.092 125.5655) (width 0.2) (layer "B.Cu") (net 20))
 (segment (start 163.092 104.9217) (end 163.3799 104.9217) (width 0.2) (layer "B.Cu") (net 20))
 (segment (start 166.8226 124.3749) (end 165.632 125.5655) (width 0.2) (layer "B.Cu") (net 18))
 (segment (start 165.632 129.8672) (end 165.632 125.5655) (width 0.2) (layer "B.Cu") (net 18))
 (segment (start 166.8226 105.8244) (end 166.8226 124.3749) (width 0.2) (layer "B.Cu") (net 18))
 (segment (start 165.632 103.77) (end 165.632 104.9217) (width 0.2) (layer "B.Cu") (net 18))
 (segment (start 165.9199 104.9217) (end 166.8226 105.8244) (width 0.2) (layer "B.Cu") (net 18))
 (segment (start 165.632 104.9217) (end 165.9199 104.9217) (width 0.2) (layer "B.Cu") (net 18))
 (segment (start 168.172 103.77) (end 168.172 104.9217) (width 0.2) (layer "B.Cu") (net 16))
 (segment (start 169.3626 124.3749) (end 168.172 125.5655) (width 0.2) (layer "B.Cu") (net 16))
 (segment (start 168.172 129.8672) (end 168.172 125.5655) (width 0.2) (layer "B.Cu") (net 16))
 (segment (start 168.172 104.9217) (end 168.4599 104.9217) (width 0.2) (layer "B.Cu") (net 16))
 (segment (start 169.3626 105.8244) (end 169.3626 124.3749) (width 0.2) (layer "B.Cu") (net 16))
 (segment (start 168.4599 104.9217) (end 169.3626 105.8244) (width 0.2) (layer "B.Cu") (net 16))
 (segment (start 190.2685 110.5067) (end 190.2685 121.4673) (width 0.2) (layer "B.Cu") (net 3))
 (segment (start 187.1037 107.3419) (end 190.2685 110.5067) (width 0.2) (layer "B.Cu") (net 3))
 (segment (start 187.1037 105.7854) (end 187.1037 107.3419) (width 0.2) (layer "B.Cu") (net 3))
 (segment (start 185.952 129.8672) (end 185.952 125.5655) (width 0.2) (layer "B.Cu") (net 3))
 (segment (start 186.24 104.9217) (end 187.1037 105.7854) (width 0.2) (layer "B.Cu") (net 3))
 (segment (start 190.2685 121.4673) (end 186.1703 125.5655) (width 0.2) (layer "B.Cu") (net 3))
 (segment (start 185.952 103.77) (end 185.952 104.9217) (width 0.2) (layer "B.Cu") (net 3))
 (segment (start 185.952 104.9217) (end 186.24 104.9217) (width 0.2) (layer "B.Cu") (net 3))
 (segment (start 186.1703 125.5655) (end 185.952 125.5655) (width 0.2) (layer "B.Cu") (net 3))
 (segment (start 188.492 103.77) (end 188.492 104.9217) (width 0.2) (layer "B.Cu") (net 1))
 (segment (start 188.7799 104.9217) (end 188.492 104.9217) (width 0.2) (layer "B.Cu") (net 1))
 (segment (start 188.492 129.8672) (end 188.492 125.5655) (width 0.2) (layer "B.Cu") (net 1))
 (segment (start 188.492 125.5655) (end 190.6958 123.3617) (width 0.2) (layer "B.Cu") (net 1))
 (segment (start 190.6958 106.8376) (end 188.7799 104.9217) (width 0.2) (layer "B.Cu") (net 1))
 (segment (start 190.6958 123.3617) (end 190.6958 106.8376) (width 0.2) (layer "B.Cu") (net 1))
 (segment (start 182.0626 124.3749) (end 180.872 125.5655) (width 0.2) (layer "B.Cu") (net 7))
 (segment (start 180.872 103.77) (end 180.872 104.9217) (width 0.2) (layer "B.Cu") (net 7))
 (segment (start 180.872 129.8672) (end 180.872 125.5655) (width 0.2) (layer "B.Cu") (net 7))
 (segment (start 181.1599 104.9217) (end 182.0626 105.8244) (width 0.2) (layer "B.Cu") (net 7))
 (segment (start 182.0626 105.8244) (end 182.0626 124.3749) (width 0.2) (layer "B.Cu") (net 7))
 (segment (start 180.872 104.9217) (end 181.1599 104.9217) (width 0.2) (layer "B.Cu") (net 7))
 (segment (start 179.4893 105.7911) (end 179.4893 124.4082) (width 0.2) (layer "B.Cu") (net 9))
 (segment (start 178.332 103.77) (end 178.332 104.9217) (width 0.2) (layer "B.Cu") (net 9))
 (segment (start 178.332 104.9217) (end 178.6199 104.9217) (width 0.2) (layer "B.Cu") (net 9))
 (segment (start 178.332 129.8672) (end 178.332 125.5655) (width 0.2) (layer "B.Cu") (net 9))
 (segment (start 179.4893 124.4082) (end 178.332 125.5655) (width 0.2) (layer "B.Cu") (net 9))
 (segment (start 178.6199 104.9217) (end 179.4893 105.7911) (width 0.2) (layer "B.Cu") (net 9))
 (segment (start 176.0605 104.9217) (end 175.792 104.9217) (width 0.2) (layer "B.Cu") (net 11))
 (segment (start 175.792 103.77) (end 175.792 104.9217) (width 0.2) (layer "B.Cu") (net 11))
 (segment (start 176.9533 124.4042) (end 176.9533 105.8145) (width 0.2) (layer "B.Cu") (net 11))
 (segment (start 175.792 125.5655) (end 176.9533 124.4042) (width 0.2) (layer "B.Cu") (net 11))
 (segment (start 175.792 129.8672) (end 175.792 125.5655) (width 0.2) (layer "B.Cu") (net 11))
 (segment (start 176.9533 105.8145) (end 176.0605 104.9217) (width 0.2) (layer "B.Cu") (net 11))
 (segment (start 174.4133 124.4042) (end 174.4133 105.8145) (width 0.2) (layer "B.Cu") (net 13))
 (segment (start 173.252 103.77) (end 173.252 104.9217) (width 0.2) (layer "B.Cu") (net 13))
 (segment (start 173.252 129.8672) (end 173.252 125.5655) (width 0.2) (layer "B.Cu") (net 13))
 (segment (start 174.4133 105.8145) (end 173.5205 104.9217) (width 0.2) (layer "B.Cu") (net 13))
 (segment (start 173.5205 104.9217) (end 173.252 104.9217) (width 0.2) (layer "B.Cu") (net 13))
 (segment (start 173.252 125.5655) (end 174.4133 124.4042) (width 0.2) (layer "B.Cu") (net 13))
 (segment (start 171.8733 124.4042) (end 170.712 125.5655) (width 0.2) (layer "B.Cu") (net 15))
 (segment (start 170.712 129.8672) (end 170.712 125.5655) (width 0.2) (layer "B.Cu") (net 15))
 (segment (start 170.712 104.9217) (end 170.9805 104.9217) (width 0.2) (layer "B.Cu") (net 15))
 (segment (start 170.9805 104.9217) (end 171.8733 105.8145) (width 0.2) (layer "B.Cu") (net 15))
 (segment (start 171.8733 105.8145) (end 171.8733 124.4042) (width 0.2) (layer "B.Cu") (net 15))
 (segment (start 170.712 103.77) (end 170.712 104.9217) (width 0.2) (layer "B.Cu") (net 15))
 (segment (start 126.7402 104.9217) (end 126.3506 105.3113) (width 0.2) (layer "B.Cu") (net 45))
 (segment (start 126.3506 124.3841) (end 127.532 125.5655) (width 0.2) (layer "B.Cu") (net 45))
 (segment (start 126.3506 105.3113) (end 126.3506 124.3841) (width 0.2) (layer "B.Cu") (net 45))
 (segment (start 127.532 104.9217) (end 126.7402 104.9217) (width 0.2) (layer "B.Cu") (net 45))
 (segment (start 127.532 129.8672) (end 127.532 125.5655) (width 0.2) (layer "B.Cu") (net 45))
 (segment (start 127.532 103.77) (end 127.532 104.9217) (width 0.2) (layer "B.Cu") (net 45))
 (segment (start 137.692 106.31) (end 137.692 129.8672) (width 0.2) (layer "F.Cu") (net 41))
 (segment (start 173.252 106.31) (end 173.252 129.8672) (width 0.2) (layer "F.Cu") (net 14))
 (segment (start 175.792 106.31) (end 175.792 129.8672) (width 0.2) (layer "F.Cu") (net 12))
 (segment (start 178.332 106.31) (end 178.332 129.8672) (width 0.2) (layer "F.Cu") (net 10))
 (segment (start 180.872 106.31) (end 180.872 129.8672) (width 0.2) (layer "F.Cu") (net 8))
 (segment (start 183.412 106.31) (end 183.412 129.8672) (width 0.2) (layer "F.Cu") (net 6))
 (segment (start 185.952 129.8672) (end 185.952 125.5655) (width 0.2) (layer "F.Cu") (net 4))
 (segment (start 186.5066 125.0109) (end 185.952 125.5655) (width 0.2) (layer "F.Cu") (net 4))
 (segment (start 186.5066 124.3486) (end 186.5066 125.0109) (width 0.2) (layer "F.Cu") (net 4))
 (via (at 186.5066 124.3486) (size 0.6) (drill 0.3) (layers "F.Cu" "B.Cu") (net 4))
 (segment (start 185.952 113.5643) (end 189.8668 117.4791) (width 0.2) (layer "B.Cu") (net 4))
 (segment (start 189.8668 120.9884) (end 186.5066 124.3486) (width 0.2) (layer "B.Cu") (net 4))
 (segment (start 185.952 106.31) (end 185.952 113.5643) (width 0.2) (layer "B.Cu") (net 4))
 (segment (start 189.8668 117.4791) (end 189.8668 120.9884) (width 0.2) (layer "B.Cu") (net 4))
 (segment (start 189.8848 124.1727) (end 188.492 125.5655) (width 0.2) (layer "F.Cu") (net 2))
 (segment (start 188.492 107.4617) (end 189.8848 108.8545) (width 0.2) (layer "F.Cu") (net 2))
 (segment (start 189.8848 108.8545) (end 189.8848 124.1727) (width 0.2) (layer "F.Cu") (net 2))
 (segment (start 188.492 129.8672) (end 188.492 125.5655) (width 0.2) (layer "F.Cu") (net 2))
 (segment (start 188.492 106.31) (end 188.492 107.4617) (width 0.2) (layer "F.Cu") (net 2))
 (segment (start 135.152 129.8672) (end 135.152 125.5655) (width 0.2) (layer "B.Cu") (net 40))
 (segment (start 137.692 103.77) (end 137.692 104.9217) (width 0.2) (layer "B.Cu") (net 40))
 (segment (start 138.8533 105.8145) (end 137.9605 104.9217) (width 0.2) (layer "B.Cu") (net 40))
 (segment (start 136.3426 124.3749) (end 135.152 125.5655) (width 0.2) (layer "B.Cu") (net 40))
 (segment (start 135.152 103.77) (end 135.152 104.9217) (width 0.2) (layer "B.Cu") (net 40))
 (segment (start 135.4399 104.9217) (end 136.3426 105.8244) (width 0.2) (layer "B.Cu") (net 40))
 (segment (start 138.8533 124.4042) (end 138.8533 105.8145) (width 0.2) (layer "B.Cu") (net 40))
 (segment (start 137.692 129.8672) (end 137.692 125.5655) (width 0.2) (layer "B.Cu") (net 40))
 (segment (start 137.9605 104.9217) (end 137.692 104.9217) (width 0.2) (layer "B.Cu") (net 40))
 (segment (start 136.3426 105.8244) (end 136.3426 124.3749) (width 0.2) (layer "B.Cu") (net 40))
 (segment (start 137.692 125.5655) (end 138.8533 124.4042) (width 0.2) (layer "B.Cu") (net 40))
 (segment (start 135.152 104.9217) (end 135.4399 104.9217) (width 0.2) (layer "B.Cu") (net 40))
 (segment (start 135.147 125.147) (end 134.5 124.5) (width 0.2) (layer "F.Cu") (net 42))
 (segment (start 132.612 124.888) (end 132.612 129.867) (width 0.2) (layer "F.Cu") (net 42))
 (segment (start 135.147 129.36) (end 135.147 127.8376) (width 0.2) (layer "F.Cu") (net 42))
 (segment (start 132.612 129.867) (end 132.612 129.8672) (width 0.2) (layer "F.Cu") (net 42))
 (segment (start 135.147 127.8376) (end 135.147 125.147) (width 0.2) (layer "F.Cu") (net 42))
 (segment (start 133 124.5) (end 132.612 124.888) (width 0.2) (layer "F.Cu") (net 42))
 (segment (start 135.1465 127.8381) (end 135.1465 129.3598) (width 0.2) (layer "F.Cu") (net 42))
 (segment (start 135.147 127.8376) (end 135.1465 127.8381) (width 0.2) (layer "F.Cu") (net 42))
 (segment (start 134.5 124.5) (end 133 124.5) (width 0.2) (layer "F.Cu") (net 42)))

